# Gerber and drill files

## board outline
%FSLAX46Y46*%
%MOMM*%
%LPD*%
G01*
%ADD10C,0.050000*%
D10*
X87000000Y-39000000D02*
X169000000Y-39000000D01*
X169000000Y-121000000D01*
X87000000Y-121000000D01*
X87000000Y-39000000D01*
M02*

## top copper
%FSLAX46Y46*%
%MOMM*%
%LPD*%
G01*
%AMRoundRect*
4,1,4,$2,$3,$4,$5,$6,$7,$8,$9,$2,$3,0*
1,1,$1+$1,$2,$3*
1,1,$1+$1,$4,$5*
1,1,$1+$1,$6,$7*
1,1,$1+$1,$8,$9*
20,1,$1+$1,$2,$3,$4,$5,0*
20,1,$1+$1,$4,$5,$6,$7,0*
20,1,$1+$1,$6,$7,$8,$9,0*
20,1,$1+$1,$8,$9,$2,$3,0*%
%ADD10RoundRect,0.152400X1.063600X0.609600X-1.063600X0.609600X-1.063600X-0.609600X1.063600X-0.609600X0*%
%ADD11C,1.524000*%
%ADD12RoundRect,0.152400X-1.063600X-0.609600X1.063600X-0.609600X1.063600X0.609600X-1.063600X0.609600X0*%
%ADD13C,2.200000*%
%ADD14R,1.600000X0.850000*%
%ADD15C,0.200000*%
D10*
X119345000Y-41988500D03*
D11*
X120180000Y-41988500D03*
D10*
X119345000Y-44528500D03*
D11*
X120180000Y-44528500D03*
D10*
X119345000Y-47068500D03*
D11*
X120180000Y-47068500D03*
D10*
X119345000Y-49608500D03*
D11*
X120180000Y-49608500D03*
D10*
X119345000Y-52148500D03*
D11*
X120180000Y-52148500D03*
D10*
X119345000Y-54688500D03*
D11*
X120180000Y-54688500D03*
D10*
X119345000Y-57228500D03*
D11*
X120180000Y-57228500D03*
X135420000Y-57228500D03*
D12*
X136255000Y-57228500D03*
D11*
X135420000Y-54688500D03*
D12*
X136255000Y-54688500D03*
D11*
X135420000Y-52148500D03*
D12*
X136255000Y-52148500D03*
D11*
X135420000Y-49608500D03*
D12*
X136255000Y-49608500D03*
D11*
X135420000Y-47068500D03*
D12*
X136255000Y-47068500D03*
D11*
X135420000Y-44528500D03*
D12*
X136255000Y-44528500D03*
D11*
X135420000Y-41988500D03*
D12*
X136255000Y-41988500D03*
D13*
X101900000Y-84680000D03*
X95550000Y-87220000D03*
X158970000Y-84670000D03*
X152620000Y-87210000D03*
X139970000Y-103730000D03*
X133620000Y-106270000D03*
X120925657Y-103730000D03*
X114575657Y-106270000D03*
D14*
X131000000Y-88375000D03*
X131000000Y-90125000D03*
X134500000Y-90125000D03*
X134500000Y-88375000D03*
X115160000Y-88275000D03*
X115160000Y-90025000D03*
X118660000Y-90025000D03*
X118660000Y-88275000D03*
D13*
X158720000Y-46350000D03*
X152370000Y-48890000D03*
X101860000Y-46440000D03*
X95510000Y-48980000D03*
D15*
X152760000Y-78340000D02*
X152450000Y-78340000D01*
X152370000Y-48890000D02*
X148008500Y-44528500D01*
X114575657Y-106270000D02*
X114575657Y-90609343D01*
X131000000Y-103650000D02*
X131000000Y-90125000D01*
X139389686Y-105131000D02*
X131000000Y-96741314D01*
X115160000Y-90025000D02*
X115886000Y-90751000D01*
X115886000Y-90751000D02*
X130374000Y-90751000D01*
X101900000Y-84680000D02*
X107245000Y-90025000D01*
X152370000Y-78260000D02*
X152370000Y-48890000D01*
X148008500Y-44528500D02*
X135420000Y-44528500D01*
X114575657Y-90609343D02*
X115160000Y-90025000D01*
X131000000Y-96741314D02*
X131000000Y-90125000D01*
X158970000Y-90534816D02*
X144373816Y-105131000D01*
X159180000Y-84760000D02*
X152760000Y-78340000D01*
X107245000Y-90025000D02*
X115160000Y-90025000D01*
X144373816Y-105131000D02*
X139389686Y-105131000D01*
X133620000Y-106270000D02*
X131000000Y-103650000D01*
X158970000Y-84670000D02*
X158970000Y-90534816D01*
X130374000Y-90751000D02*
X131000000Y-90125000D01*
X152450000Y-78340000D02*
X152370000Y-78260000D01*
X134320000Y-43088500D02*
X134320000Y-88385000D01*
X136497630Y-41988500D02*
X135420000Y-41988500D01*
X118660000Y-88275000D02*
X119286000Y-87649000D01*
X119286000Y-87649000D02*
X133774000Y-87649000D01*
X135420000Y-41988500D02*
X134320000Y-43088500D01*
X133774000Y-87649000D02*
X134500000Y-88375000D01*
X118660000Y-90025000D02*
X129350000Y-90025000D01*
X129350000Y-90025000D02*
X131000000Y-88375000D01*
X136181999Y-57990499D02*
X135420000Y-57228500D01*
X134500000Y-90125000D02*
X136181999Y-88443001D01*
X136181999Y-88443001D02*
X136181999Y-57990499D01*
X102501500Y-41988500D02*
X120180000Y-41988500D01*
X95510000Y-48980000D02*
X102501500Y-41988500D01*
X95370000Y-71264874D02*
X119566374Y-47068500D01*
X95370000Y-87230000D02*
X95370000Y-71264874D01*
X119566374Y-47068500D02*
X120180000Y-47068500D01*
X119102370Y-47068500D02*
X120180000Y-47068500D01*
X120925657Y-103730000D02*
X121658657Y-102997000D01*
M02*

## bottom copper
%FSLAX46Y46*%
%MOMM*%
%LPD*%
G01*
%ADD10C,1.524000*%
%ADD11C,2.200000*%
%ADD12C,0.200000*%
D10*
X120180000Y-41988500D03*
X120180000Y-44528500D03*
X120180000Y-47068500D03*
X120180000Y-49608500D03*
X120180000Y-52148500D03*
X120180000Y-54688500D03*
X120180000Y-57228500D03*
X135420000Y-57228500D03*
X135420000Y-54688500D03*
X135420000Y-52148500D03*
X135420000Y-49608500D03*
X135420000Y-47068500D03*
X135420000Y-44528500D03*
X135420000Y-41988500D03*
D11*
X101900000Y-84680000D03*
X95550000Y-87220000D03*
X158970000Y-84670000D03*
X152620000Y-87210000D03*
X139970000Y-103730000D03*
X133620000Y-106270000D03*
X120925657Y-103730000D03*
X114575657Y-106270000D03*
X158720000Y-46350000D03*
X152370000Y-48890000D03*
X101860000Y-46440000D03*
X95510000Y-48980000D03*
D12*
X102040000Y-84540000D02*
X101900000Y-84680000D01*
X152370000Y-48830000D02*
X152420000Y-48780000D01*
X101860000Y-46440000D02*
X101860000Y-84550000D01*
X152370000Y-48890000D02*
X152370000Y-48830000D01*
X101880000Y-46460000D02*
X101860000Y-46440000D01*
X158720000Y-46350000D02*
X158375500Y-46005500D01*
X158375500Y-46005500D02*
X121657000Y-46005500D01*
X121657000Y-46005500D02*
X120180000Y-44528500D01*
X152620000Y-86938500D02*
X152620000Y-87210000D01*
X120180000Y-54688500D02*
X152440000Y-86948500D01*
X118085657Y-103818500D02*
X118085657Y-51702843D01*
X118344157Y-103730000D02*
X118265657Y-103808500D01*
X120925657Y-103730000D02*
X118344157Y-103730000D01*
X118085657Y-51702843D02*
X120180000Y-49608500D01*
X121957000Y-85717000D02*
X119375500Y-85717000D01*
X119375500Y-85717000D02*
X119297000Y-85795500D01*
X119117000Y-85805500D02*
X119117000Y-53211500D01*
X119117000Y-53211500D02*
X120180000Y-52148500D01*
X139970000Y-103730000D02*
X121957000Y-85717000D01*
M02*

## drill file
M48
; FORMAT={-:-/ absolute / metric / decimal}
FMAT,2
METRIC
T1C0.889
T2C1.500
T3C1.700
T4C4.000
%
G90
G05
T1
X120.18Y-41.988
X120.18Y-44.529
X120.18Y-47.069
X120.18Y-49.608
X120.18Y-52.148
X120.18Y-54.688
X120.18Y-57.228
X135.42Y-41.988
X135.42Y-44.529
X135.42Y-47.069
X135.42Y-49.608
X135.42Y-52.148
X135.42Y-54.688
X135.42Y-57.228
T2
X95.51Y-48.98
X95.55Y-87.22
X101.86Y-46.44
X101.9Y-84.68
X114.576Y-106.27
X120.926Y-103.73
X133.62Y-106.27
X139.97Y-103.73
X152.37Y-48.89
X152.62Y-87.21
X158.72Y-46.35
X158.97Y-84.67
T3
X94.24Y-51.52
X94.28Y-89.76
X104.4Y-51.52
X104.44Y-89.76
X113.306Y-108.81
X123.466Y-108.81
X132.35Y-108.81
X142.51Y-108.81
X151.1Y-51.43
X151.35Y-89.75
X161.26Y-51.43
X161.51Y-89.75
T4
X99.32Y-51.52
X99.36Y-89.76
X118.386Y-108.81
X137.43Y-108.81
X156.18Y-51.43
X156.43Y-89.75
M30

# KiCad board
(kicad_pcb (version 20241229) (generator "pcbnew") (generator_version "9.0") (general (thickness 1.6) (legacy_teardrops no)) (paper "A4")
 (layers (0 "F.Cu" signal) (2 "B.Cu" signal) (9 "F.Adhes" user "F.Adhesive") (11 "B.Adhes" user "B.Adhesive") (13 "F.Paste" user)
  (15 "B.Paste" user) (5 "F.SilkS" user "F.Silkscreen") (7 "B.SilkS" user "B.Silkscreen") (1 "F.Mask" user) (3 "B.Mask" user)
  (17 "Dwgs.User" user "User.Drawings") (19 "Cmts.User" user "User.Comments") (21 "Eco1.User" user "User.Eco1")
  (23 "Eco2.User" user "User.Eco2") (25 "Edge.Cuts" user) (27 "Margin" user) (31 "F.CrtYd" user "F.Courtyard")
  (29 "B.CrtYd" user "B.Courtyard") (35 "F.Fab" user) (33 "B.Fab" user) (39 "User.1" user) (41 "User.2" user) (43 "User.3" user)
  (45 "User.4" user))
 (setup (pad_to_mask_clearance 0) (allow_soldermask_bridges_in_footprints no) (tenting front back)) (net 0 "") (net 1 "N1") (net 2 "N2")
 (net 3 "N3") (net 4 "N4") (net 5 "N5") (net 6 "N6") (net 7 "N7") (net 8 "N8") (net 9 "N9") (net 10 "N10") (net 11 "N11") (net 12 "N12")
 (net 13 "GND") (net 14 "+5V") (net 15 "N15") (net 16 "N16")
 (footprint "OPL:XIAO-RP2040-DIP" (layer "F.Cu") (at 127.8 49.6085)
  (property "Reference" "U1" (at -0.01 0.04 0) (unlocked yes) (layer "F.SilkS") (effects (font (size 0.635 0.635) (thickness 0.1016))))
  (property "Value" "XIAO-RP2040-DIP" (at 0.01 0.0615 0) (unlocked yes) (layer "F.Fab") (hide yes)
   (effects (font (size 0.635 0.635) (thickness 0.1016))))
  (pad "1" smd roundrect (at -8.455 -7.62 180) (size 2.432 1.524) (layers "F.Cu" "F.Mask") (roundrect_rratio 0.1) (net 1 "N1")
   (thermal_bridge_angle 45))
  (pad "1" thru_hole circle (at -7.62 -7.62 180) (size 1.524 1.524) (drill 0.889) (layers "*.Cu" "*.Mask") (remove_unused_layers no)
   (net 1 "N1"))
  (pad "2" smd roundrect (at -8.455 -5.08 180) (size 2.432 1.524) (layers "F.Cu" "F.Mask") (roundrect_rratio 0.1) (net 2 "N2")
   (thermal_bridge_angle 45))
  (pad "2" thru_hole circle (at -7.62 -5.08 180) (size 1.524 1.524) (drill 0.889) (layers "*.Cu" "*.Mask") (remove_unused_layers no)
   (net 2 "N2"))
  (pad "3" smd roundrect (at -8.455 -2.54 180) (size 2.432 1.524) (layers "F.Cu" "F.Mask") (roundrect_rratio 0.1) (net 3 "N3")
   (thermal_bridge_angle 45))
  (pad "3" thru_hole circle (at -7.62 -2.54 180) (size 1.524 1.524) (drill 0.889) (layers "*.Cu" "*.Mask") (remove_unused_layers no)
   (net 3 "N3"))
  (pad "4" smd roundrect (at -8.455 0 180) (size 2.432 1.524) (layers "F.Cu" "F.Mask") (roundrect_rratio 0.1) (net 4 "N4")
   (thermal_bridge_angle 45))
  (pad "4" thru_hole circle (at -7.62 0 180) (size 1.524 1.524) (drill 0.889) (layers "*.Cu" "*.Mask") (remove_unused_layers no)
   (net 4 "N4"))
  (pad "5" smd roundrect (at -8.455 2.54 180) (size 2.432 1.524) (layers "F.Cu" "F.Mask") (roundrect_rratio 0.1) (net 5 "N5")
   (thermal_bridge_angle 45))
  (pad "5" thru_hole circle (at -7.62 2.54 180) (size 1.524 1.524) (drill 0.889) (layers "*.Cu" "*.Mask") (remove_unused_layers no)
   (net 5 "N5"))
  (pad "6" smd roundrect (at -8.455 5.08 180) (size 2.432 1.524) (layers "F.Cu" "F.Mask") (roundrect_rratio 0.1) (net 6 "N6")
   (thermal_bridge_angle 45))
  (pad "6" thru_hole circle (at -7.62 5.08 180) (size 1.524 1.524) (drill 0.889) (layers "*.Cu" "*.Mask") (remove_unused_layers no)
   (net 6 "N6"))
  (pad "7" smd roundrect (at -8.455 7.62 180) (size 2.432 1.524) (layers "F.Cu" "F.Mask") (roundrect_rratio 0.1) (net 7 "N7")
   (thermal_bridge_angle 45))
  (pad "7" thru_hole circle (at -7.62 7.62 180) (size 1.524 1.524) (drill 0.889) (layers "*.Cu" "*.Mask") (remove_unused_layers no)
   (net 7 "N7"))
  (pad "8" thru_hole circle (at 7.62 7.62) (size 1.524 1.524) (drill 0.889) (layers "*.Cu" "*.Mask") (remove_unused_layers no) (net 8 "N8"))
  (pad "8" smd roundrect (at 8.455 7.62) (size 2.432 1.524) (layers "F.Cu" "F.Mask") (roundrect_rratio 0.1) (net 8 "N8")
   (thermal_bridge_angle 45))
  (pad "9" thru_hole circle (at 7.62 5.08) (size 1.524 1.524) (drill 0.889) (layers "*.Cu" "*.Mask") (remove_unused_layers no) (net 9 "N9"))
  (pad "9" smd roundrect (at 8.455 5.08) (size 2.432 1.524) (layers "F.Cu" "F.Mask") (roundrect_rratio 0.1) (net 9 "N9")
   (thermal_bridge_angle 45))
  (pad "10" thru_hole circle (at 7.62 2.54) (size 1.524 1.524) (drill 0.889) (layers "*.Cu" "*.Mask") (remove_unused_layers no)
   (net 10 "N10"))
  (pad "10" smd roundrect (at 8.455 2.54) (size 2.432 1.524) (layers "F.Cu" "F.Mask") (roundrect_rratio 0.1) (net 10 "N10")
   (thermal_bridge_angle 45))
  (pad "11" thru_hole circle (at 7.62 0) (size 1.524 1.524) (drill 0.889) (layers "*.Cu" "*.Mask") (remove_unused_layers no) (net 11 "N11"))
  (pad "11" smd roundrect (at 8.455 0) (size 2.432 1.524) (layers "F.Cu" "F.Mask") (roundrect_rratio 0.1) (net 11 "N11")
   (thermal_bridge_angle 45))
  (pad "12" thru_hole circle (at 7.62 -2.54) (size 1.524 1.524) (drill 0.889) (layers "*.Cu" "*.Mask") (remove_unused_layers no)
   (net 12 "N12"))
  (pad "12" smd roundrect (at 8.455 -2.54) (size 2.432 1.524) (layers "F.Cu" "F.Mask") (roundrect_rratio 0.1) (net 12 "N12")
   (thermal_bridge_angle 45))
  (pad "13" thru_hole circle (at 7.62 -5.08) (size 1.524 1.524) (drill 0.889) (layers "*.Cu" "*.Mask") (remove_unused_layers no)
   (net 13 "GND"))
  (pad "13" smd roundrect (at 8.455 -5.08) (size 2.432 1.524) (layers "F.Cu" "F.Mask") (roundrect_rratio 0.1) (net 13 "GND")
   (thermal_bridge_angle 45))
  (pad "14" thru_hole circle (at 7.62 -7.62) (size 1.524 1.524) (drill 0.889) (layers "*.Cu" "*.Mask") (remove_unused_layers no)
   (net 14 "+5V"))
  (pad "14" smd roundrect (at 8.455 -7.62) (size 2.432 1.524) (layers "F.Cu" "F.Mask") (roundrect_rratio 0.1) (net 14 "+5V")
   (thermal_bridge_angle 45)))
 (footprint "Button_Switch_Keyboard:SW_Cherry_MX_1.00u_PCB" (layer "F.Cu") (at 101.9 84.68)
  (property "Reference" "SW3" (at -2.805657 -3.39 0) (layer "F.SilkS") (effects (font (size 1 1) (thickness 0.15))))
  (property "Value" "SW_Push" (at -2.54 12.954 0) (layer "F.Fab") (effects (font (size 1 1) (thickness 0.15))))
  (pad "" np_thru_hole circle (at -7.62 5.08) (size 1.7 1.7) (drill 1.7) (layers "*.Cu" "*.Mask"))
  (pad "" np_thru_hole circle (at -2.54 5.08) (size 4 4) (drill 4) (layers "*.Cu" "*.Mask"))
  (pad "" np_thru_hole circle (at 2.54 5.08) (size 1.7 1.7) (drill 1.7) (layers "*.Cu" "*.Mask"))
  (pad "1" thru_hole circle (at 0 0) (size 2.2 2.2) (drill 1.5) (layers "*.Cu" "*.Mask") (remove_unused_layers no) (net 13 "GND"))
  (pad "2" thru_hole circle (at -6.35 2.54) (size 2.2 2.2) (drill 1.5) (layers "*.Cu" "*.Mask") (remove_unused_layers no) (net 3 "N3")))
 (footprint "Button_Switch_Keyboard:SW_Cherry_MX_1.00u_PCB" (layer "F.Cu") (at 158.97 84.67)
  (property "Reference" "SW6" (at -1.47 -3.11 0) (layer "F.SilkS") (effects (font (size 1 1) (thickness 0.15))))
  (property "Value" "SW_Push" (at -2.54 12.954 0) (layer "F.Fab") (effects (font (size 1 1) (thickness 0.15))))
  (pad "" np_thru_hole circle (at -7.62 5.08) (size 1.7 1.7) (drill 1.7) (layers "*.Cu" "*.Mask"))
  (pad "" np_thru_hole circle (at -2.54 5.08) (size 4 4) (drill 4) (layers "*.Cu" "*.Mask"))
  (pad "" np_thru_hole circle (at 2.54 5.08) (size 1.7 1.7) (drill 1.7) (layers "*.Cu" "*.Mask"))
  (pad "1" thru_hole circle (at 0 0) (size 2.2 2.2) (drill 1.5) (layers "*.Cu" "*.Mask") (remove_unused_layers no) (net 13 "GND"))
  (pad "2" thru_hole circle (at -6.35 2.54) (size 2.2 2.2) (drill 1.5) (layers "*.Cu" "*.Mask") (remove_unused_layers no) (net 6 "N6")))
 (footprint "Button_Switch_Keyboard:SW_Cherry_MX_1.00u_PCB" (layer "F.Cu") (at 139.97 103.73)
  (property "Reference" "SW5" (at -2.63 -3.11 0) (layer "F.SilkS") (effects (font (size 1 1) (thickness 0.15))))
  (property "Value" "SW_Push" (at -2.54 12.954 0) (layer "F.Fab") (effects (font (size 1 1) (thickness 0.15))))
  (pad "" np_thru_hole circle (at -7.62 5.08) (size 1.7 1.7) (drill 1.7) (layers "*.Cu" "*.Mask"))
  (pad "" np_thru_hole circle (at -2.54 5.08) (size 4 4) (drill 4) (layers "*.Cu" "*.Mask"))
  (pad "" np_thru_hole circle (at 2.54 5.08) (size 1.7 1.7) (drill 1.7) (layers "*.Cu" "*.Mask"))
  (pad "1" thru_hole circle (at 0 0) (size 2.2 2.2) (drill 1.5) (layers "*.Cu" "*.Mask") (remove_unused_layers no) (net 5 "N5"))
  (pad "2" thru_hole circle (at -6.35 2.54) (size 2.2 2.2) (drill 1.5) (layers "*.Cu" "*.Mask") (remove_unused_layers no) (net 13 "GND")))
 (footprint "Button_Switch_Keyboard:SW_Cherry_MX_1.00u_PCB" (layer "F.Cu") (at 120.925657 103.73)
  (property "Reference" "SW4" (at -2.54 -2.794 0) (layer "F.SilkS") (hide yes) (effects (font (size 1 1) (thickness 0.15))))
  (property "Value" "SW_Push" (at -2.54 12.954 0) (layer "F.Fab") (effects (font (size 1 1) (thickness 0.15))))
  (pad "" np_thru_hole circle (at -7.62 5.08) (size 1.7 1.7) (drill 1.7) (layers "*.Cu" "*.Mask"))
  (pad "" np_thru_hole circle (at -2.54 5.08) (size 4 4) (drill 4) (layers "*.Cu" "*.Mask"))
  (pad "" np_thru_hole circle (at 2.54 5.08) (size 1.7 1.7) (drill 1.7) (layers "*.Cu" "*.Mask"))
  (pad "1" thru_hole circle (at 0 0) (size 2.2 2.2) (drill 1.5) (layers "*.Cu" "*.Mask") (remove_unused_layers no) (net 4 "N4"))
  (pad "2" thru_hole circle (at -6.35 2.54) (size 2.2 2.2) (drill 1.5) (layers "*.Cu" "*.Mask") (remove_unused_layers no) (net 13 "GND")))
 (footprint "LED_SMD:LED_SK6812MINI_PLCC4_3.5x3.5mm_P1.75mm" (layer "F.Cu") (at 132.75 89.25)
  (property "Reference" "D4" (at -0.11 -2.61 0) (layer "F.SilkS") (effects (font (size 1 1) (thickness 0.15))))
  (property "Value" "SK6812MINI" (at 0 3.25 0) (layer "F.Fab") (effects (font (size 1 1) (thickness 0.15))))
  (pad "1" smd rect (at -1.75 -0.875) (size 1.6 0.85) (layers "F.Cu" "F.Mask" "F.Paste") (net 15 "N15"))
  (pad "2" smd rect (at -1.75 0.875) (size 1.6 0.85) (layers "F.Cu" "F.Mask" "F.Paste") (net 13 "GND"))
  (pad "3" smd rect (at 1.75 0.875) (size 1.6 0.85) (layers "F.Cu" "F.Mask" "F.Paste") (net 8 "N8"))
  (pad "4" smd rect (at 1.75 -0.875) (size 1.6 0.85) (layers "F.Cu" "F.Mask" "F.Paste") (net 14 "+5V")))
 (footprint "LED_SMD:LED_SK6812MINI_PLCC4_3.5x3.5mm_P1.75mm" (layer "F.Cu") (at 116.91 89.15)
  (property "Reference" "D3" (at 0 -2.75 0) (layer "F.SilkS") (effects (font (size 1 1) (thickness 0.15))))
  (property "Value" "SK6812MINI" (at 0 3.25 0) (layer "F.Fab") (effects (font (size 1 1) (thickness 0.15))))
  (pad "1" smd rect (at -1.75 -0.875) (size 1.6 0.85) (layers "F.Cu" "F.Mask" "F.Paste") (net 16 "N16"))
  (pad "2" smd rect (at -1.75 0.875) (size 1.6 0.85) (layers "F.Cu" "F.Mask" "F.Paste") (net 13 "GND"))
  (pad "3" smd rect (at 1.75 0.875) (size 1.6 0.85) (layers "F.Cu" "F.Mask" "F.Paste") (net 15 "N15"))
  (pad "4" smd rect (at 1.75 -0.875) (size 1.6 0.85) (layers "F.Cu" "F.Mask" "F.Paste") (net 14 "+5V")))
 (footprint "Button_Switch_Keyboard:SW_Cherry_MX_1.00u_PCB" (layer "F.Cu") (at 158.72 46.35)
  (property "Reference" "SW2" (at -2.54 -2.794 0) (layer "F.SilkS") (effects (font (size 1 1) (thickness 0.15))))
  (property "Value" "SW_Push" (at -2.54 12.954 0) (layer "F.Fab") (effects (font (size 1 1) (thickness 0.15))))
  (pad "" np_thru_hole circle (at -7.62 5.08) (size 1.7 1.7) (drill 1.7) (layers "*.Cu" "*.Mask"))
  (pad "" np_thru_hole circle (at -2.54 5.08) (size 4 4) (drill 4) (layers "*.Cu" "*.Mask"))
  (pad "" np_thru_hole circle (at 2.54 5.08) (size 1.7 1.7) (drill 1.7) (layers "*.Cu" "*.Mask"))
  (pad "1" thru_hole circle (at 0 0) (size 2.2 2.2) (drill 1.5) (layers "*.Cu" "*.Mask") (remove_unused_layers no) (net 2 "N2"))
  (pad "2" thru_hole circle (at -6.35 2.54) (size 2.2 2.2) (drill 1.5) (layers "*.Cu" "*.Mask") (remove_unused_layers no) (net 13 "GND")))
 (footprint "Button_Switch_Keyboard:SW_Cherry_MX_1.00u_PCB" (layer "F.Cu") (at 101.86 46.44)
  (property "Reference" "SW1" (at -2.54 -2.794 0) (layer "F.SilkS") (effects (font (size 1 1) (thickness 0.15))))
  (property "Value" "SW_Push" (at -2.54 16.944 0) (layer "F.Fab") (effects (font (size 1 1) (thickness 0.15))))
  (pad "" np_thru_hole circle (at -7.62 5.08) (size 1.7 1.7) (drill 1.7) (layers "*.Cu" "*.Mask"))
  (pad "" np_thru_hole circle (at -2.54 5.08) (size 4 4) (drill 4) (layers "*.Cu" "*.Mask"))
  (pad "" np_thru_hole circle (at 2.54 5.08) (size 1.7 1.7) (drill 1.7) (layers "*.Cu" "*.Mask"))
  (pad "1" thru_hole circle (at 0 0) (size 2.2 2.2) (drill 1.5) (layers "*.Cu" "*.Mask") (remove_unused_layers no) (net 13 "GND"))
  (pad "2" thru_hole circle (at -6.35 2.54) (size 2.2 2.2) (drill 1.5) (layers "*.Cu" "*.Mask") (remove_unused_layers no) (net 1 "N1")))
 (gr_rect (start 87 39) (end 169 121) (stroke (width 0.05) (type solid)) (fill no) (layer "Edge.Cuts"))
 (segment (start 152.76 78.34) (end 152.45 78.34) (width 0.2) (layer "F.Cu") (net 13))
 (segment (start 152.37 48.89) (end 148.0085 44.5285) (width 0.2) (layer "F.Cu") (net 13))
 (segment (start 114.575657 106.27) (end 114.575657 90.609343) (width 0.2) (layer "F.Cu") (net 13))
 (segment (start 131 103.65) (end 131 90.125) (width 0.2) (layer "F.Cu") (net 13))
 (segment (start 139.389686 105.131) (end 131 96.741314) (width 0.2) (layer "F.Cu") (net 13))
 (segment (start 115.16 90.025) (end 115.886 90.751) (width 0.2) (layer "F.Cu") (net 13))
 (segment (start 115.886 90.751) (end 130.374 90.751) (width 0.2) (layer "F.Cu") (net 13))
 (segment (start 101.9 84.68) (end 107.245 90.025) (width 0.2) (layer "F.Cu") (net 13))
 (segment (start 152.37 78.26) (end 152.37 48.89) (width 0.2) (layer "F.Cu") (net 13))
 (segment (start 148.0085 44.5285) (end 135.42 44.5285) (width 0.2) (layer "F.Cu") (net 13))
 (segment (start 114.575657 90.609343) (end 115.16 90.025) (width 0.2) (layer "F.Cu") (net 13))
 (segment (start 131 96.741314) (end 131 90.125) (width 0.2) (layer "F.Cu") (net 13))
 (segment (start 158.97 90.534816) (end 144.373816 105.131) (width 0.2) (layer "F.Cu") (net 13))
 (segment (start 159.18 84.76) (end 152.76 78.34) (width 0.2) (layer "F.Cu") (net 13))
 (segment (start 107.245 90.025) (end 115.16 90.025) (width 0.2) (layer "F.Cu") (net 13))
 (segment (start 144.373816 105.131) (end 139.389686 105.131) (width 0.2) (layer "F.Cu") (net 13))
 (segment (start 133.62 106.27) (end 131 103.65) (width 0.2) (layer "F.Cu") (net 13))
 (segment (start 158.97 84.67) (end 158.97 90.534816) (width 0.2) (layer "F.Cu") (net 13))
 (segment (start 130.374 90.751) (end 131 90.125) (width 0.2) (layer "F.Cu") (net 13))
 (segment (start 152.45 78.34) (end 152.37 78.26) (width 0.2) (layer "F.Cu") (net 13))
 (segment (start 102.04 84.54) (end 101.9 84.68) (width 0.2) (layer "B.Cu") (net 13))
 (segment (start 152.37 48.83) (end 152.42 48.78) (width 0.2) (layer "B.Cu") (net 13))
 (segment (start 101.86 46.44) (end 101.86 84.55) (width 0.2) (layer "B.Cu") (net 13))
 (segment (start 152.37 48.89) (end 152.37 48.83) (width 0.2) (layer "B.Cu") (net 13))
 (segment (start 101.88 46.46) (end 101.86 46.44) (width 0.2) (layer "B.Cu") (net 13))
 (segment (start 134.32 43.0885) (end 134.32 88.385) (width 0.2) (layer "F.Cu") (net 14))
 (segment (start 136.49763 41.9885) (end 135.42 41.9885) (width 0.2) (layer "F.Cu") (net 14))
 (segment (start 118.66 88.275) (end 119.286 87.649) (width 0.2) (layer "F.Cu") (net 14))
 (segment (start 119.286 87.649) (end 133.774 87.649) (width 0.2) (layer "F.Cu") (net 14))
 (segment (start 135.42 41.9885) (end 134.32 43.0885) (width 0.2) (layer "F.Cu") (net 14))
 (segment (start 133.774 87.649) (end 134.5 88.375) (width 0.2) (layer "F.Cu") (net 14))
 (segment (start 118.66 90.025) (end 129.35 90.025) (width 0.2) (layer "F.Cu") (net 15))
 (segment (start 129.35 90.025) (end 131 88.375) (width 0.2) (layer "F.Cu") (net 15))
 (segment (start 136.181999 57.990499) (end 135.42 57.2285) (width 0.2) (layer "F.Cu") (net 8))
 (segment (start 134.5 90.125) (end 136.181999 88.443001) (width 0.2) (layer "F.Cu") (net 8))
 (segment (start 136.181999 88.443001) (end 136.181999 57.990499) (width 0.2) (layer "F.Cu") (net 8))
 (segment (start 102.5015 41.9885) (end 120.18 41.9885) (width 0.2) (layer "F.Cu") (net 1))
 (segment (start 95.51 48.98) (end 102.5015 41.9885) (width 0.2) (layer "F.Cu") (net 1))
 (segment (start 158.72 46.35) (end 158.3755 46.0055) (width 0.2) (layer "B.Cu") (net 2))
 (segment (start 158.3755 46.0055) (end 121.657 46.0055) (width 0.2) (layer "B.Cu") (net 2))
 (segment (start 121.657 46.0055) (end 120.18 44.5285) (width 0.2) (layer "B.Cu") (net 2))
 (segment (start 95.37 71.264874) (end 119.566374 47.0685) (width 0.2) (layer "F.Cu") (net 3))
 (segment (start 95.37 87.23) (end 95.37 71.264874) (width 0.2) (layer "F.Cu") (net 3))
 (segment (start 119.566374 47.0685) (end 120.18 47.0685) (width 0.2) (layer "F.Cu") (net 3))
 (segment (start 119.10237 47.0685) (end 120.18 47.0685) (width 0.2) (layer "F.Cu") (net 3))
 (segment (start 152.62 86.9385) (end 152.62 87.21) (width 0.2) (layer "B.Cu") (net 6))
 (segment (start 120.18 54.6885) (end 152.44 86.9485) (width 0.2) (layer "B.Cu") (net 6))
 (segment (start 120.925657 103.73) (end 121.658657 102.997) (width 0.2) (layer "F.Cu") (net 4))
 (segment (start 118.085657 103.8185) (end 118.085657 51.702843) (width 0.2) (layer "B.Cu") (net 4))
 (segment (start 118.344157 103.73) (end 118.265657 103.8085) (width 0.2) (layer "B.Cu") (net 4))
 (segment (start 120.925657 103.73) (end 118.344157 103.73) (width 0.2) (layer "B.Cu") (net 4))
 (segment (start 118.085657 51.702843) (end 120.18 49.6085) (width 0.2) (layer "B.Cu") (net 4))
 (segment (start 121.957 85.717) (end 119.3755 85.717) (width 0.2) (layer "B.Cu") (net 5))
 (segment (start 119.3755 85.717) (end 119.297 85.7955) (width 0.2) (layer "B.Cu") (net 5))
 (segment (start 119.117 85.8055) (end 119.117 53.2115) (width 0.2) (layer "B.Cu") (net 5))
 (segment (start 119.117 53.2115) (end 120.18 52.1485) (width 0.2) (layer "B.Cu") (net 5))
 (segment (start 139.97 103.73) (end 121.957 85.717) (width 0.2) (layer "B.Cu") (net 5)))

